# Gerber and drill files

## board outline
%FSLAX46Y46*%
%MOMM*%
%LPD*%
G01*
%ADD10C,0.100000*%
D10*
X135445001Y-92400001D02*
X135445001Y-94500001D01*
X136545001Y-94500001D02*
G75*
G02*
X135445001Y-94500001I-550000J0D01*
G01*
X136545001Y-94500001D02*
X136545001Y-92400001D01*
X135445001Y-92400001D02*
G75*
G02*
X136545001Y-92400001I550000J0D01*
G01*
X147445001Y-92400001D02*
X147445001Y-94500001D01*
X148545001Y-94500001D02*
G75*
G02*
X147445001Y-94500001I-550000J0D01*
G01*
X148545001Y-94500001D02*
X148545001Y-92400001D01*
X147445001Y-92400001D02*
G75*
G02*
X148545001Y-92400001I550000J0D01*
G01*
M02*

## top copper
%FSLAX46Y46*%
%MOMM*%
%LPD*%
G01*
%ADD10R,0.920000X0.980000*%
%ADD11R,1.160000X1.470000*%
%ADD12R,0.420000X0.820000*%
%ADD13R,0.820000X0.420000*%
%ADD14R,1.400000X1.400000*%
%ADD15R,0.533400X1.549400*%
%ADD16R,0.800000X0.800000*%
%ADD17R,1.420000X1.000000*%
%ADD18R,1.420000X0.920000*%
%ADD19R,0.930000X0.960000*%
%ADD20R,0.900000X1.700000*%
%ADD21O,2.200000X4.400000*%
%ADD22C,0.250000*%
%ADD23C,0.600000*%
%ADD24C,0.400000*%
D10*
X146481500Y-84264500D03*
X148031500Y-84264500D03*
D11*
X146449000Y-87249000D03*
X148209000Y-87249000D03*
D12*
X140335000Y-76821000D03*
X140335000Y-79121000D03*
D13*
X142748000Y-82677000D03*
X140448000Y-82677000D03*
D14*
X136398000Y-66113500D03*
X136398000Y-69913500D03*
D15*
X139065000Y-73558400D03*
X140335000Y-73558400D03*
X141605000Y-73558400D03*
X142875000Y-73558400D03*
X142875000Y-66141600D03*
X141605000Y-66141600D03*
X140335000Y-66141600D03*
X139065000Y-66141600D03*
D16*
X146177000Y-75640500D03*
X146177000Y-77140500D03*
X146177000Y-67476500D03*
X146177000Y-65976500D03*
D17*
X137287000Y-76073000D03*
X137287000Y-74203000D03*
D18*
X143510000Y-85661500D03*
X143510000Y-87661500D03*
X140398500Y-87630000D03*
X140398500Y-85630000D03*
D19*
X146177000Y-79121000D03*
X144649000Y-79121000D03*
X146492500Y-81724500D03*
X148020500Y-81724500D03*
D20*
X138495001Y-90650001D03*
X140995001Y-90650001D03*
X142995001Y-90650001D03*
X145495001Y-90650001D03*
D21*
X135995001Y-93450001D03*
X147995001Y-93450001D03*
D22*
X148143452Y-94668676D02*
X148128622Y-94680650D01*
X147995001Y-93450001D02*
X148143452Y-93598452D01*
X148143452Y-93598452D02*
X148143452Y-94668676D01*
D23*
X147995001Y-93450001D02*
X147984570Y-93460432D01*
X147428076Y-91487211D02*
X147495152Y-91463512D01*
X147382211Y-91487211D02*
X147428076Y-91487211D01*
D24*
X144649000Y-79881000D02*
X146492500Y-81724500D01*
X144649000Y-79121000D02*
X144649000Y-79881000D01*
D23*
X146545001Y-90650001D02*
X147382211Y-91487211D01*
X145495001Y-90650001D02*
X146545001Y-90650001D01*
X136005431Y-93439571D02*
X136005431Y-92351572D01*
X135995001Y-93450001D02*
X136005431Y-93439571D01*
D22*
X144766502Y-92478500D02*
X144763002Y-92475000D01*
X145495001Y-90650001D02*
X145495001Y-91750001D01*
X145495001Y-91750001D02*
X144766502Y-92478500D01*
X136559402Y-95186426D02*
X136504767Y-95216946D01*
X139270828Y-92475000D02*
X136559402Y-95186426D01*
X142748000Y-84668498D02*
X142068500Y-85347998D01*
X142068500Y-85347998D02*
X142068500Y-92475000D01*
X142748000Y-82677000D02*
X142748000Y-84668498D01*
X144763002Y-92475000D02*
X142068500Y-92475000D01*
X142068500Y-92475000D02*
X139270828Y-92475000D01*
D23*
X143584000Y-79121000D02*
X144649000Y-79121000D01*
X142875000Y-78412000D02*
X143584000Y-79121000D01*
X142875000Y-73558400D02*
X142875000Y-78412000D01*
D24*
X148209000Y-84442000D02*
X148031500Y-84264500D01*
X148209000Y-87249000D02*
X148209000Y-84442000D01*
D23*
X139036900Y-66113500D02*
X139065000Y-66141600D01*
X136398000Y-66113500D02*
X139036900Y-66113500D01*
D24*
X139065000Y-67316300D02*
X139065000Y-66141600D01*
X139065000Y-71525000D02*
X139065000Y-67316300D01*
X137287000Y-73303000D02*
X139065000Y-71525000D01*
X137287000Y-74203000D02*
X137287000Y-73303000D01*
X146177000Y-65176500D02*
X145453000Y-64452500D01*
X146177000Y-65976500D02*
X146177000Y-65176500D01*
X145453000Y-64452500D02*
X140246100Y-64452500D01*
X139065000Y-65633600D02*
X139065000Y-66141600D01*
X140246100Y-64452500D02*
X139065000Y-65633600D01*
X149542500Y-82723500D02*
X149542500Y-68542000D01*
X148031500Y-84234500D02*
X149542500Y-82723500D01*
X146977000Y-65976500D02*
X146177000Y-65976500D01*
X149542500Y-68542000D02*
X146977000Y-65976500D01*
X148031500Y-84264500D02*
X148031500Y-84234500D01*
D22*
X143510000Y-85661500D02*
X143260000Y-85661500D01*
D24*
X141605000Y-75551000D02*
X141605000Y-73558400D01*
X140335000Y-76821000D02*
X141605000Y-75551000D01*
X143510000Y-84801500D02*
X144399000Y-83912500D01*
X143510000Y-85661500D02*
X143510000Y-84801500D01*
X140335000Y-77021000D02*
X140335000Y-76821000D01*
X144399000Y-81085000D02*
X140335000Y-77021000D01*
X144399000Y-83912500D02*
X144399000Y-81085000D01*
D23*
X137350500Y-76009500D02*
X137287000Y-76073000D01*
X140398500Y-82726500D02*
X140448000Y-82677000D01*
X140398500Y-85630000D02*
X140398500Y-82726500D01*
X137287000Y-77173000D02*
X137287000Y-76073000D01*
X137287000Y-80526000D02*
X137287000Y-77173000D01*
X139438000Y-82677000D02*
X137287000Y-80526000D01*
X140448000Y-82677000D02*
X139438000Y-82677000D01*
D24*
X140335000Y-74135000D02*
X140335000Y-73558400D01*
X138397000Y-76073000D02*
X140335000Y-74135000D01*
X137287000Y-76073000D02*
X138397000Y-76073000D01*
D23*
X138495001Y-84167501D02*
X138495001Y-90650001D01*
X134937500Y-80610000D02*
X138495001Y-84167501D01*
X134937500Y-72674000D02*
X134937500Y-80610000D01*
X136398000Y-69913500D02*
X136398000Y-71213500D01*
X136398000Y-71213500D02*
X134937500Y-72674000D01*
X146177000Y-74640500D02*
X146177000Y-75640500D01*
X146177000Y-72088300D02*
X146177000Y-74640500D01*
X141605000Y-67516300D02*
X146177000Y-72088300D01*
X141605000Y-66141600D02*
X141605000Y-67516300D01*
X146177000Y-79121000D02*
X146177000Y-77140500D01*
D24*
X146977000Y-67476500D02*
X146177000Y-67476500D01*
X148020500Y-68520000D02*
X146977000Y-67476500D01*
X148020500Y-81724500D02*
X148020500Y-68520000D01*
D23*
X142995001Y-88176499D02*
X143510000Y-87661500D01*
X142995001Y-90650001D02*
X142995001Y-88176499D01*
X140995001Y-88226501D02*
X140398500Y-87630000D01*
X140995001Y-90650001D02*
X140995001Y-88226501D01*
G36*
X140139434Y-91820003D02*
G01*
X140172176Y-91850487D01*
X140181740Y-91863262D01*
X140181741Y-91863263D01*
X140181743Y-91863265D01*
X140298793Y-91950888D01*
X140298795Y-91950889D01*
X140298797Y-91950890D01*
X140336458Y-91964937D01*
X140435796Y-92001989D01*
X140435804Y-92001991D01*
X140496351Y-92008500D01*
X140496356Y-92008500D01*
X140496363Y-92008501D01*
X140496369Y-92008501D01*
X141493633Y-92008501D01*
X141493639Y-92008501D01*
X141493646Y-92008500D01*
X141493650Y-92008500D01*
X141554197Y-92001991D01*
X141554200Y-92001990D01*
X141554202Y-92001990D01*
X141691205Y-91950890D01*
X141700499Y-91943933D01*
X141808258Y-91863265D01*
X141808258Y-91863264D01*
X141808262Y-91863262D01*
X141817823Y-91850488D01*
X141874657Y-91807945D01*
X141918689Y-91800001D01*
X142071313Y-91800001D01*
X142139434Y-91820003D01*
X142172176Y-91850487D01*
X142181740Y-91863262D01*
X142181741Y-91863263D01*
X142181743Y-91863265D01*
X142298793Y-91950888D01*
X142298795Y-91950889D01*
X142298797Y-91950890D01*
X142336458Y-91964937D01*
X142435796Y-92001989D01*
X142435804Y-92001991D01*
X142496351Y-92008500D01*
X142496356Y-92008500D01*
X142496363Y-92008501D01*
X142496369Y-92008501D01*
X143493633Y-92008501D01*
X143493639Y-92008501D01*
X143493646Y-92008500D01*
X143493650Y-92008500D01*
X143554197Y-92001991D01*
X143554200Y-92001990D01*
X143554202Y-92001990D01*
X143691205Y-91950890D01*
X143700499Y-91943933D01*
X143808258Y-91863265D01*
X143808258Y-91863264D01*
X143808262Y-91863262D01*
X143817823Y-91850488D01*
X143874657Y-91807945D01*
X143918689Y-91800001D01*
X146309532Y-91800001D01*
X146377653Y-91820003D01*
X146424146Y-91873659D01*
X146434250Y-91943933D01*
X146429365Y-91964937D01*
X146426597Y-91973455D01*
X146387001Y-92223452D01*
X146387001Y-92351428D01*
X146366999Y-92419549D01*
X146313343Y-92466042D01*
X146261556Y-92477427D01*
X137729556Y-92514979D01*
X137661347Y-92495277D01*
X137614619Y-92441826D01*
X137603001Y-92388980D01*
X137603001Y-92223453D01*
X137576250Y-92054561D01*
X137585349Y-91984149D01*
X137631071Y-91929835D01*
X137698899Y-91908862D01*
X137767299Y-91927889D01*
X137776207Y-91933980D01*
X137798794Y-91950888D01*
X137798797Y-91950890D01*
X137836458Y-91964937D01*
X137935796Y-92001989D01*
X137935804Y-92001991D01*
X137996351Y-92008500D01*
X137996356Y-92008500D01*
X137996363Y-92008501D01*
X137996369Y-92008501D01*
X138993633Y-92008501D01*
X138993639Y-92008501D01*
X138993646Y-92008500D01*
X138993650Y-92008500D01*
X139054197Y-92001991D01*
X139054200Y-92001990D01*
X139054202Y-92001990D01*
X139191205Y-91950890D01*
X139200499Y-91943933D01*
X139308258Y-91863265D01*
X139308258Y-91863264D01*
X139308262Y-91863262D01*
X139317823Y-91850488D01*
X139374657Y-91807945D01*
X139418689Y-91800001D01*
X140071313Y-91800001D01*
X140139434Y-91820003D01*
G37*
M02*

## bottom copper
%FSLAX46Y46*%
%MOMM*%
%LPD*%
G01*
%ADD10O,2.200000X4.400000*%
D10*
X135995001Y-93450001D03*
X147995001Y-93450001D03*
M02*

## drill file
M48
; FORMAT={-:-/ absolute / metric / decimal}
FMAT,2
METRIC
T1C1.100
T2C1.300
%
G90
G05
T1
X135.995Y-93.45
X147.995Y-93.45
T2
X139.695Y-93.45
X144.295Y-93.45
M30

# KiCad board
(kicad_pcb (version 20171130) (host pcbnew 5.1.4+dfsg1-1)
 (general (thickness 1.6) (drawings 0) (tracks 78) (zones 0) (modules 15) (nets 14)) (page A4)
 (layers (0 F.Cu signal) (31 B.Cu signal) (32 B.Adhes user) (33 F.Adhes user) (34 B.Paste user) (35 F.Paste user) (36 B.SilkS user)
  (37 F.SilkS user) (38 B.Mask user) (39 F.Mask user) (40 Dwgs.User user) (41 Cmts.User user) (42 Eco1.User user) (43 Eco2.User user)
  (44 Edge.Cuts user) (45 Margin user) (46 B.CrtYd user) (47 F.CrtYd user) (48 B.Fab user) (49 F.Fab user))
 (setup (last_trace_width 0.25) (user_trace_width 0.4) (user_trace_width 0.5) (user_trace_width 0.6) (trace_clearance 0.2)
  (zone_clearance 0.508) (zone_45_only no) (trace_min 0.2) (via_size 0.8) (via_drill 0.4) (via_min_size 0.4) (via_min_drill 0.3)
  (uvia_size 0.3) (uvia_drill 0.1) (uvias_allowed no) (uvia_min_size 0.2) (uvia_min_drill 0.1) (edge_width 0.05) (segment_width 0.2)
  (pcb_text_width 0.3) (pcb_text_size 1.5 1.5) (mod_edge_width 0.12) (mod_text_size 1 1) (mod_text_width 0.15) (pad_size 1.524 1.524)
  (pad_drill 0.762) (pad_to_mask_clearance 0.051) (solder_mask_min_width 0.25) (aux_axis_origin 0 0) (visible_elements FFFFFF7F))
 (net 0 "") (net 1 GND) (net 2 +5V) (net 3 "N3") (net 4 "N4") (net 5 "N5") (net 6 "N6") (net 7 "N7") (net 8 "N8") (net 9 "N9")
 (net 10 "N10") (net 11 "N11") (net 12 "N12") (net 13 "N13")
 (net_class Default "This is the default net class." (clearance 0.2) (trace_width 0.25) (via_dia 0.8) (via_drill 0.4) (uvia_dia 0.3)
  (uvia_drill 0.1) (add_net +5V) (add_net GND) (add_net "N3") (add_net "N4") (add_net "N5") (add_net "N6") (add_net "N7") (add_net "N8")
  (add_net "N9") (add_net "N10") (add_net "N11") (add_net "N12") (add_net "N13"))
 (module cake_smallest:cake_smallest (layer F.Cu) (at 146.304 73.152 90)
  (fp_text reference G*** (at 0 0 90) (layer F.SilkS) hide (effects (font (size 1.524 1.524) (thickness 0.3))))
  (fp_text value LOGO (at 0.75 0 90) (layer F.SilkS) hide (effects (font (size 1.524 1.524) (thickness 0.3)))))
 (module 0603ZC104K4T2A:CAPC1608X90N (layer F.Cu) (at 147.2565 84.2645)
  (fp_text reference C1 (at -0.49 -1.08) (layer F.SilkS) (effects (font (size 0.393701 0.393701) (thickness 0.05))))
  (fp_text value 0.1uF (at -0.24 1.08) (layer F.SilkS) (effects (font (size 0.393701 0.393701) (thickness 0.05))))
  (pad 1 smd rect (at -0.775 0) (size 0.92 0.98) (layers F.Cu F.Paste F.Mask) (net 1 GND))
  (pad 2 smd rect (at 0.775 0) (size 0.92 0.98) (layers F.Cu F.Paste F.Mask) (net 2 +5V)))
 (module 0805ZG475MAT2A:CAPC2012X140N (layer F.Cu) (at 147.329 87.249)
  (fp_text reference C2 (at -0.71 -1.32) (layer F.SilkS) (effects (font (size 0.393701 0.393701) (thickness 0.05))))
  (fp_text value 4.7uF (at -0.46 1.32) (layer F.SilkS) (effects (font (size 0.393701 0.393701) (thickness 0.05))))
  (pad 1 smd rect (at -0.88 0) (size 1.16 1.47) (layers F.Cu F.Paste F.Mask) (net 1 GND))
  (pad 2 smd rect (at 0.88 0) (size 1.16 1.47) (layers F.Cu F.Paste F.Mask) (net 2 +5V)))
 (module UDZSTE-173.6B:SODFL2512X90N (layer F.Cu) (at 140.335 77.971 270)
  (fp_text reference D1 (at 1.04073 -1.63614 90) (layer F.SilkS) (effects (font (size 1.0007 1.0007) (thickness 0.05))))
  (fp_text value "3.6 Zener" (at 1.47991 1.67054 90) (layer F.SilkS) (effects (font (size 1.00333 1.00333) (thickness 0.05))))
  (pad C smd rect (at -1.15 0 270) (size 0.82 0.42) (layers F.Cu F.Paste F.Mask) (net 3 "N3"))
  (pad A smd rect (at 1.15 0 270) (size 0.82 0.42) (layers F.Cu F.Paste F.Mask) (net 1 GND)))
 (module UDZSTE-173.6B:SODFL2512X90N (layer F.Cu) (at 141.598 82.677)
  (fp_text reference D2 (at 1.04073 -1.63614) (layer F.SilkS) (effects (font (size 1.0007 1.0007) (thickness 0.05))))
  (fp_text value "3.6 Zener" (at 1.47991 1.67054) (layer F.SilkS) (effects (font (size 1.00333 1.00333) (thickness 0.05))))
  (pad A smd rect (at 1.15 0) (size 0.82 0.42) (layers F.Cu F.Paste F.Mask) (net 1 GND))
  (pad C smd rect (at -1.15 0) (size 0.82 0.42) (layers F.Cu F.Paste F.Mask) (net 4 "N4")))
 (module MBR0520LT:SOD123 (layer F.Cu) (at 136.398 68.0135 270)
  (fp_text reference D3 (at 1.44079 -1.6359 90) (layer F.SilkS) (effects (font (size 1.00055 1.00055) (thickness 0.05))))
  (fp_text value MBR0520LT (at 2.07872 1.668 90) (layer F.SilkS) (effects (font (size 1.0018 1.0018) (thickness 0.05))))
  (pad C smd rect (at -1.9 0 270) (size 1.4 1.4) (layers F.Cu F.Paste F.Mask) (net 2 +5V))
  (pad A smd rect (at 1.9 0 270) (size 1.4 1.4) (layers F.Cu F.Paste F.Mask) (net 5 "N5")))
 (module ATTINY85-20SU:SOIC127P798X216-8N (layer F.Cu) (at 140.97 69.85 90)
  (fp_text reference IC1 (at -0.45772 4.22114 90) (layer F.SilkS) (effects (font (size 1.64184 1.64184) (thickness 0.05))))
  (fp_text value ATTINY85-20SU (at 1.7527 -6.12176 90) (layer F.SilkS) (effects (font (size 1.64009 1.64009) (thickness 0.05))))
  (pad 1 smd rect (at -3.7084 -1.905 90) (size 1.5494 0.5334) (layers F.Cu F.Paste F.Mask) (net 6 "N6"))
  (pad 2 smd rect (at -3.7084 -0.635 90) (size 1.5494 0.5334) (layers F.Cu F.Paste F.Mask) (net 4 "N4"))
  (pad 3 smd rect (at -3.7084 0.635 90) (size 1.5494 0.5334) (layers F.Cu F.Paste F.Mask) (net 3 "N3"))
  (pad 4 smd rect (at -3.7084 1.905 90) (size 1.5494 0.5334) (layers F.Cu F.Paste F.Mask) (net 1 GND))
  (pad 5 smd rect (at 3.7084 1.905 90) (size 1.5494 0.5334) (layers F.Cu F.Paste F.Mask) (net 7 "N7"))
  (pad 6 smd rect (at 3.7084 0.635 90) (size 1.5494 0.5334) (layers F.Cu F.Paste F.Mask) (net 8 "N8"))
  (pad 7 smd rect (at 3.7084 -0.635 90) (size 1.5494 0.5334) (layers F.Cu F.Paste F.Mask) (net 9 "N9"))
  (pad 8 smd rect (at 3.7084 -1.905 90) (size 1.5494 0.5334) (layers F.Cu F.Paste F.Mask) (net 2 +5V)))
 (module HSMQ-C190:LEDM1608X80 (layer F.Cu) (at 146.177 76.3905 90)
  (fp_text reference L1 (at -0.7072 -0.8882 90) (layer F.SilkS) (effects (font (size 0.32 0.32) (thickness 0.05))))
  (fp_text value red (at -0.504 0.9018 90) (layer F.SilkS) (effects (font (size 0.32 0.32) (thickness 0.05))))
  (pad A smd rect (at 0.75 0 180) (size 0.8 0.8) (layers F.Cu F.Paste F.Mask) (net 8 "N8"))
  (pad C smd rect (at -0.75 0 180) (size 0.8 0.8) (layers F.Cu F.Paste F.Mask) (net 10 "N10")))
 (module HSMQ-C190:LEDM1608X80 (layer F.Cu) (at 146.177 66.7265 90)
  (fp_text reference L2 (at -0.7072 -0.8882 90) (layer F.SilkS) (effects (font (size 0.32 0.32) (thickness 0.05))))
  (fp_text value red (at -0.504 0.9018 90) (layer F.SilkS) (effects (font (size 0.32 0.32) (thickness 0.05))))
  (pad C smd rect (at -0.75 0 180) (size 0.8 0.8) (layers F.Cu F.Paste F.Mask) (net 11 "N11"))
  (pad A smd rect (at 0.75 0 180) (size 0.8 0.8) (layers F.Cu F.Paste F.Mask) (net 2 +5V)))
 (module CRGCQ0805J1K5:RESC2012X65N (layer F.Cu) (at 137.287 75.138 90)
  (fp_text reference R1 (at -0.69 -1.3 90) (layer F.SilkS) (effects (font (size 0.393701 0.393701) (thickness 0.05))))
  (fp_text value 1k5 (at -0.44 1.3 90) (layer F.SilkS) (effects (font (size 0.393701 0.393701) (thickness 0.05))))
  (pad 1 smd rect (at -0.935 0 90) (size 1 1.42) (layers F.Cu F.Paste F.Mask) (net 4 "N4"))
  (pad 2 smd rect (at 0.935 0 90) (size 1 1.42) (layers F.Cu F.Paste F.Mask) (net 2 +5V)))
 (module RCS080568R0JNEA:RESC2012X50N (layer F.Cu) (at 143.51 86.6615 90)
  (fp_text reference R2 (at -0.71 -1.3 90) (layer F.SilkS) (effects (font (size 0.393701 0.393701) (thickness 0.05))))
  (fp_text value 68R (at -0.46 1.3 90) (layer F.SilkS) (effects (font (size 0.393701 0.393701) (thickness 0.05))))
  (pad 2 smd rect (at 1 0 90) (size 0.92 1.42) (layers F.Cu F.Paste F.Mask) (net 3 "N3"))
  (pad 1 smd rect (at -1 0 90) (size 0.92 1.42) (layers F.Cu F.Paste F.Mask) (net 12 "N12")))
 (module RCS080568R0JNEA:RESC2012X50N (layer F.Cu) (at 140.3985 86.63 90)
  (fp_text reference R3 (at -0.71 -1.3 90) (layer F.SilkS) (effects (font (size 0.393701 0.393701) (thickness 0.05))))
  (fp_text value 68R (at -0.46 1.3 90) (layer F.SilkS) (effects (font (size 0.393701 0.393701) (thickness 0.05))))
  (pad 1 smd rect (at -1 0 90) (size 0.92 1.42) (layers F.Cu F.Paste F.Mask) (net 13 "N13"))
  (pad 2 smd rect (at 1 0 90) (size 0.92 1.42) (layers F.Cu F.Paste F.Mask) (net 4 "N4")))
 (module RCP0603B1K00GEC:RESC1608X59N (layer F.Cu) (at 145.413 79.121)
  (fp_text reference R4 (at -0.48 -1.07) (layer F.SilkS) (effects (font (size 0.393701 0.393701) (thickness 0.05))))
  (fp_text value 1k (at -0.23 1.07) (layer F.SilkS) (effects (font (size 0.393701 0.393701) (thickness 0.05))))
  (pad 2 smd rect (at 0.764 0) (size 0.93 0.96) (layers F.Cu F.Paste F.Mask) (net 10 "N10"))
  (pad 1 smd rect (at -0.764 0) (size 0.93 0.96) (layers F.Cu F.Paste F.Mask) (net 1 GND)))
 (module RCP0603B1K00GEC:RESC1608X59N (layer F.Cu) (at 147.2565 81.7245)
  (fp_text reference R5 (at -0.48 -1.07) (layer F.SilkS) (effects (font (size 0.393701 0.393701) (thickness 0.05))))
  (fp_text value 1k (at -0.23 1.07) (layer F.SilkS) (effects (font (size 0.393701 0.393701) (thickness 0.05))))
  (pad 1 smd rect (at -0.764 0) (size 0.93 0.96) (layers F.Cu F.Paste F.Mask) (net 1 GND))
  (pad 2 smd rect (at 0.764 0) (size 0.93 0.96) (layers F.Cu F.Paste F.Mask) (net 11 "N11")))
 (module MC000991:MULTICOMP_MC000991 (layer F.Cu) (at 141.995001 93.450001)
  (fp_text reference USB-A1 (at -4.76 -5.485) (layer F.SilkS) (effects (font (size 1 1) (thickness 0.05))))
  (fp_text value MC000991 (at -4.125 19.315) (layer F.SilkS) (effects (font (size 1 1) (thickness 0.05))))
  (fp_line (start -6.55 -1.05) (end -6.55 1.05) (layer Edge.Cuts) (width 0.1))
  (fp_arc (start -6 1.05) (end -5.45 1.05) (angle 180) (layer Edge.Cuts) (width 0.1))
  (fp_line (start -5.45 1.05) (end -5.45 -1.05) (layer Edge.Cuts) (width 0.1))
  (fp_arc (start -6 -1.05) (end -6.55 -1.05) (angle 180) (layer Edge.Cuts) (width 0.1))
  (fp_line (start 5.45 -1.05) (end 5.45 1.05) (layer Edge.Cuts) (width 0.1))
  (fp_arc (start 6 1.05) (end 6.55 1.05) (angle 180) (layer Edge.Cuts) (width 0.1))
  (fp_line (start 6.55 1.05) (end 6.55 -1.05) (layer Edge.Cuts) (width 0.1))
  (fp_arc (start 6 -1.05) (end 5.45 -1.05) (angle 180) (layer Edge.Cuts) (width 0.1))
  (pad 1 smd rect (at -3.5 -2.8) (size 0.9 1.7) (layers F.Cu F.Paste F.Mask) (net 5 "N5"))
  (pad 2 smd rect (at -1 -2.8) (size 0.9 1.7) (layers F.Cu F.Paste F.Mask) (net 13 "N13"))
  (pad 3 smd rect (at 1 -2.8) (size 0.9 1.7) (layers F.Cu F.Paste F.Mask) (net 12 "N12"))
  (pad 4 smd rect (at 3.5 -2.8) (size 0.9 1.7) (layers F.Cu F.Paste F.Mask) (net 1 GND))
  (pad Hole np_thru_hole circle (at 2.3 0) (size 1.3 1.3) (drill 1.3) (layers *.Cu *.Mask F.SilkS))
  (pad Hole np_thru_hole circle (at -2.3 0) (size 1.3 1.3) (drill 1.3) (layers *.Cu *.Mask F.SilkS))
  (pad S1 thru_hole oval (at -6 0 90) (size 4.4 2.2) (drill 1.1) (layers *.Cu *.Mask) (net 1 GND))
  (pad S2 thru_hole oval (at 6 0 90) (size 4.4 2.2) (drill 1.1) (layers *.Cu *.Mask) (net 1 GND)))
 (segment (start 148.143452 94.668676) (end 148.128622 94.68065) (width 0.25) (layer F.Cu) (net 1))
 (segment (start 147.995001 93.450001) (end 148.143452 93.598452) (width 0.25) (layer F.Cu) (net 1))
 (segment (start 148.143452 93.598452) (end 148.143452 94.668676) (width 0.25) (layer F.Cu) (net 1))
 (segment (start 147.995001 93.450001) (end 147.98457 93.460432) (width 0.6) (layer F.Cu) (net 1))
 (segment (start 147.428076 91.487211) (end 147.495152 91.463512) (width 0.6) (layer F.Cu) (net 1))
 (segment (start 147.382211 91.487211) (end 147.428076 91.487211) (width 0.6) (layer F.Cu) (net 1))
 (segment (start 144.649 79.881) (end 146.4925 81.7245) (width 0.4) (layer F.Cu) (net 1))
 (segment (start 144.649 79.121) (end 144.649 79.881) (width 0.4) (layer F.Cu) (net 1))
 (segment (start 146.545001 90.650001) (end 147.382211 91.487211) (width 0.6) (layer F.Cu) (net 1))
 (segment (start 145.495001 90.650001) (end 146.545001 90.650001) (width 0.6) (layer F.Cu) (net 1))
 (segment (start 136.005431 93.439571) (end 136.005431 92.351572) (width 0.6) (layer F.Cu) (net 1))
 (segment (start 135.995001 93.450001) (end 136.005431 93.439571) (width 0.6) (layer F.Cu) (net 1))
 (segment (start 144.766502 92.4785) (end 144.763002 92.475) (width 0.25) (layer F.Cu) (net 1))
 (segment (start 145.495001 90.650001) (end 145.495001 91.750001) (width 0.25) (layer F.Cu) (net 1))
 (segment (start 145.495001 91.750001) (end 144.766502 92.4785) (width 0.25) (layer F.Cu) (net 1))
 (segment (start 136.559402 95.186426) (end 136.504767 95.216946) (width 0.25) (layer F.Cu) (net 1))
 (segment (start 139.270828 92.475) (end 136.559402 95.186426) (width 0.25) (layer F.Cu) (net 1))
 (segment (start 142.748 84.668498) (end 142.0685 85.347998) (width 0.25) (layer F.Cu) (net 1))
 (segment (start 142.0685 85.347998) (end 142.0685 92.475) (width 0.25) (layer F.Cu) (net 1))
 (segment (start 142.748 82.677) (end 142.748 84.668498) (width 0.25) (layer F.Cu) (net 1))
 (segment (start 144.763002 92.475) (end 142.0685 92.475) (width 0.25) (layer F.Cu) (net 1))
 (segment (start 142.0685 92.475) (end 139.270828 92.475) (width 0.25) (layer F.Cu) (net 1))
 (segment (start 143.584 79.121) (end 144.649 79.121) (width 0.6) (layer F.Cu) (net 1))
 (segment (start 142.875 78.412) (end 143.584 79.121) (width 0.6) (layer F.Cu) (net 1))
 (segment (start 142.875 73.5584) (end 142.875 78.412) (width 0.6) (layer F.Cu) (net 1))
 (segment (start 148.209 84.442) (end 148.0315 84.2645) (width 0.4) (layer F.Cu) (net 2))
 (segment (start 148.209 87.249) (end 148.209 84.442) (width 0.4) (layer F.Cu) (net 2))
 (segment (start 139.0369 66.1135) (end 139.065 66.1416) (width 0.6) (layer F.Cu) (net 2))
 (segment (start 136.398 66.1135) (end 139.0369 66.1135) (width 0.6) (layer F.Cu) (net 2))
 (segment (start 139.065 67.3163) (end 139.065 66.1416) (width 0.4) (layer F.Cu) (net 2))
 (segment (start 139.065 71.525) (end 139.065 67.3163) (width 0.4) (layer F.Cu) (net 2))
 (segment (start 137.287 73.303) (end 139.065 71.525) (width 0.4) (layer F.Cu) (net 2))
 (segment (start 137.287 74.203) (end 137.287 73.303) (width 0.4) (layer F.Cu) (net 2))
 (segment (start 146.177 65.1765) (end 145.453 64.4525) (width 0.4) (layer F.Cu) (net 2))
 (segment (start 146.177 65.9765) (end 146.177 65.1765) (width 0.4) (layer F.Cu) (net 2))
 (segment (start 145.453 64.4525) (end 140.2461 64.4525) (width 0.4) (layer F.Cu) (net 2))
 (segment (start 139.065 65.6336) (end 139.065 66.1416) (width 0.4) (layer F.Cu) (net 2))
 (segment (start 140.2461 64.4525) (end 139.065 65.6336) (width 0.4) (layer F.Cu) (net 2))
 (segment (start 149.5425 82.7235) (end 149.5425 68.542) (width 0.4) (layer F.Cu) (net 2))
 (segment (start 148.0315 84.2345) (end 149.5425 82.7235) (width 0.4) (layer F.Cu) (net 2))
 (segment (start 146.977 65.9765) (end 146.177 65.9765) (width 0.4) (layer F.Cu) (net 2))
 (segment (start 149.5425 68.542) (end 146.977 65.9765) (width 0.4) (layer F.Cu) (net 2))
 (segment (start 148.0315 84.2645) (end 148.0315 84.2345) (width 0.4) (layer F.Cu) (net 2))
 (segment (start 143.51 85.6615) (end 143.26 85.6615) (width 0.25) (layer F.Cu) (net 3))
 (segment (start 141.605 75.551) (end 141.605 73.5584) (width 0.4) (layer F.Cu) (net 3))
 (segment (start 140.335 76.821) (end 141.605 75.551) (width 0.4) (layer F.Cu) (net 3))
 (segment (start 143.51 84.8015) (end 144.399 83.9125) (width 0.4) (layer F.Cu) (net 3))
 (segment (start 143.51 85.6615) (end 143.51 84.8015) (width 0.4) (layer F.Cu) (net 3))
 (segment (start 140.335 77.021) (end 140.335 76.821) (width 0.4) (layer F.Cu) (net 3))
 (segment (start 144.399 81.085) (end 140.335 77.021) (width 0.4) (layer F.Cu) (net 3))
 (segment (start 144.399 83.9125) (end 144.399 81.085) (width 0.4) (layer F.Cu) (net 3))
 (segment (start 137.3505 76.0095) (end 137.287 76.073) (width 0.6) (layer F.Cu) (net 4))
 (segment (start 140.3985 82.7265) (end 140.448 82.677) (width 0.6) (layer F.Cu) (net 4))
 (segment (start 140.3985 85.63) (end 140.3985 82.7265) (width 0.6) (layer F.Cu) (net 4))
 (segment (start 137.287 77.173) (end 137.287 76.073) (width 0.6) (layer F.Cu) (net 4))
 (segment (start 137.287 80.526) (end 137.287 77.173) (width 0.6) (layer F.Cu) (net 4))
 (segment (start 139.438 82.677) (end 137.287 80.526) (width 0.6) (layer F.Cu) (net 4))
 (segment (start 140.448 82.677) (end 139.438 82.677) (width 0.6) (layer F.Cu) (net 4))
 (segment (start 140.335 74.135) (end 140.335 73.5584) (width 0.4) (layer F.Cu) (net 4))
 (segment (start 138.397 76.073) (end 140.335 74.135) (width 0.4) (layer F.Cu) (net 4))
 (segment (start 137.287 76.073) (end 138.397 76.073) (width 0.4) (layer F.Cu) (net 4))
 (segment (start 138.495001 84.167501) (end 138.495001 90.650001) (width 0.6) (layer F.Cu) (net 5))
 (segment (start 134.9375 80.61) (end 138.495001 84.167501) (width 0.6) (layer F.Cu) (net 5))
 (segment (start 134.9375 72.674) (end 134.9375 80.61) (width 0.6) (layer F.Cu) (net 5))
 (segment (start 136.398 69.9135) (end 136.398 71.2135) (width 0.6) (layer F.Cu) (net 5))
 (segment (start 136.398 71.2135) (end 134.9375 72.674) (width 0.6) (layer F.Cu) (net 5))
 (segment (start 146.177 74.6405) (end 146.177 75.6405) (width 0.6) (layer F.Cu) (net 8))
 (segment (start 146.177 72.0883) (end 146.177 74.6405) (width 0.6) (layer F.Cu) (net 8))
 (segment (start 141.605 67.5163) (end 146.177 72.0883) (width 0.6) (layer F.Cu) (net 8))
 (segment (start 141.605 66.1416) (end 141.605 67.5163) (width 0.6) (layer F.Cu) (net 8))
 (segment (start 146.177 79.121) (end 146.177 77.1405) (width 0.6) (layer F.Cu) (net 10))
 (segment (start 146.977 67.4765) (end 146.177 67.4765) (width 0.4) (layer F.Cu) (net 11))
 (segment (start 148.0205 68.52) (end 146.977 67.4765) (width 0.4) (layer F.Cu) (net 11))
 (segment (start 148.0205 81.7245) (end 148.0205 68.52) (width 0.4) (layer F.Cu) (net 11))
 (segment (start 142.995001 88.176499) (end 143.51 87.6615) (width 0.6) (layer F.Cu) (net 12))
 (segment (start 142.995001 90.650001) (end 142.995001 88.176499) (width 0.6) (layer F.Cu) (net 12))
 (segment (start 140.995001 88.226501) (end 140.3985 87.63) (width 0.6) (layer F.Cu) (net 13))
 (segment (start 140.995001 90.650001) (end 140.995001 88.226501) (width 0.6) (layer F.Cu) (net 13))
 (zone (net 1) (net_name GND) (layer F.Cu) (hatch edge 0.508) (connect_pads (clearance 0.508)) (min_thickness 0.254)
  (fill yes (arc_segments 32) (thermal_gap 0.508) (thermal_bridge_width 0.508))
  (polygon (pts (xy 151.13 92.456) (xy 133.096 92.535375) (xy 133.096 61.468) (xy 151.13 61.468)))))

